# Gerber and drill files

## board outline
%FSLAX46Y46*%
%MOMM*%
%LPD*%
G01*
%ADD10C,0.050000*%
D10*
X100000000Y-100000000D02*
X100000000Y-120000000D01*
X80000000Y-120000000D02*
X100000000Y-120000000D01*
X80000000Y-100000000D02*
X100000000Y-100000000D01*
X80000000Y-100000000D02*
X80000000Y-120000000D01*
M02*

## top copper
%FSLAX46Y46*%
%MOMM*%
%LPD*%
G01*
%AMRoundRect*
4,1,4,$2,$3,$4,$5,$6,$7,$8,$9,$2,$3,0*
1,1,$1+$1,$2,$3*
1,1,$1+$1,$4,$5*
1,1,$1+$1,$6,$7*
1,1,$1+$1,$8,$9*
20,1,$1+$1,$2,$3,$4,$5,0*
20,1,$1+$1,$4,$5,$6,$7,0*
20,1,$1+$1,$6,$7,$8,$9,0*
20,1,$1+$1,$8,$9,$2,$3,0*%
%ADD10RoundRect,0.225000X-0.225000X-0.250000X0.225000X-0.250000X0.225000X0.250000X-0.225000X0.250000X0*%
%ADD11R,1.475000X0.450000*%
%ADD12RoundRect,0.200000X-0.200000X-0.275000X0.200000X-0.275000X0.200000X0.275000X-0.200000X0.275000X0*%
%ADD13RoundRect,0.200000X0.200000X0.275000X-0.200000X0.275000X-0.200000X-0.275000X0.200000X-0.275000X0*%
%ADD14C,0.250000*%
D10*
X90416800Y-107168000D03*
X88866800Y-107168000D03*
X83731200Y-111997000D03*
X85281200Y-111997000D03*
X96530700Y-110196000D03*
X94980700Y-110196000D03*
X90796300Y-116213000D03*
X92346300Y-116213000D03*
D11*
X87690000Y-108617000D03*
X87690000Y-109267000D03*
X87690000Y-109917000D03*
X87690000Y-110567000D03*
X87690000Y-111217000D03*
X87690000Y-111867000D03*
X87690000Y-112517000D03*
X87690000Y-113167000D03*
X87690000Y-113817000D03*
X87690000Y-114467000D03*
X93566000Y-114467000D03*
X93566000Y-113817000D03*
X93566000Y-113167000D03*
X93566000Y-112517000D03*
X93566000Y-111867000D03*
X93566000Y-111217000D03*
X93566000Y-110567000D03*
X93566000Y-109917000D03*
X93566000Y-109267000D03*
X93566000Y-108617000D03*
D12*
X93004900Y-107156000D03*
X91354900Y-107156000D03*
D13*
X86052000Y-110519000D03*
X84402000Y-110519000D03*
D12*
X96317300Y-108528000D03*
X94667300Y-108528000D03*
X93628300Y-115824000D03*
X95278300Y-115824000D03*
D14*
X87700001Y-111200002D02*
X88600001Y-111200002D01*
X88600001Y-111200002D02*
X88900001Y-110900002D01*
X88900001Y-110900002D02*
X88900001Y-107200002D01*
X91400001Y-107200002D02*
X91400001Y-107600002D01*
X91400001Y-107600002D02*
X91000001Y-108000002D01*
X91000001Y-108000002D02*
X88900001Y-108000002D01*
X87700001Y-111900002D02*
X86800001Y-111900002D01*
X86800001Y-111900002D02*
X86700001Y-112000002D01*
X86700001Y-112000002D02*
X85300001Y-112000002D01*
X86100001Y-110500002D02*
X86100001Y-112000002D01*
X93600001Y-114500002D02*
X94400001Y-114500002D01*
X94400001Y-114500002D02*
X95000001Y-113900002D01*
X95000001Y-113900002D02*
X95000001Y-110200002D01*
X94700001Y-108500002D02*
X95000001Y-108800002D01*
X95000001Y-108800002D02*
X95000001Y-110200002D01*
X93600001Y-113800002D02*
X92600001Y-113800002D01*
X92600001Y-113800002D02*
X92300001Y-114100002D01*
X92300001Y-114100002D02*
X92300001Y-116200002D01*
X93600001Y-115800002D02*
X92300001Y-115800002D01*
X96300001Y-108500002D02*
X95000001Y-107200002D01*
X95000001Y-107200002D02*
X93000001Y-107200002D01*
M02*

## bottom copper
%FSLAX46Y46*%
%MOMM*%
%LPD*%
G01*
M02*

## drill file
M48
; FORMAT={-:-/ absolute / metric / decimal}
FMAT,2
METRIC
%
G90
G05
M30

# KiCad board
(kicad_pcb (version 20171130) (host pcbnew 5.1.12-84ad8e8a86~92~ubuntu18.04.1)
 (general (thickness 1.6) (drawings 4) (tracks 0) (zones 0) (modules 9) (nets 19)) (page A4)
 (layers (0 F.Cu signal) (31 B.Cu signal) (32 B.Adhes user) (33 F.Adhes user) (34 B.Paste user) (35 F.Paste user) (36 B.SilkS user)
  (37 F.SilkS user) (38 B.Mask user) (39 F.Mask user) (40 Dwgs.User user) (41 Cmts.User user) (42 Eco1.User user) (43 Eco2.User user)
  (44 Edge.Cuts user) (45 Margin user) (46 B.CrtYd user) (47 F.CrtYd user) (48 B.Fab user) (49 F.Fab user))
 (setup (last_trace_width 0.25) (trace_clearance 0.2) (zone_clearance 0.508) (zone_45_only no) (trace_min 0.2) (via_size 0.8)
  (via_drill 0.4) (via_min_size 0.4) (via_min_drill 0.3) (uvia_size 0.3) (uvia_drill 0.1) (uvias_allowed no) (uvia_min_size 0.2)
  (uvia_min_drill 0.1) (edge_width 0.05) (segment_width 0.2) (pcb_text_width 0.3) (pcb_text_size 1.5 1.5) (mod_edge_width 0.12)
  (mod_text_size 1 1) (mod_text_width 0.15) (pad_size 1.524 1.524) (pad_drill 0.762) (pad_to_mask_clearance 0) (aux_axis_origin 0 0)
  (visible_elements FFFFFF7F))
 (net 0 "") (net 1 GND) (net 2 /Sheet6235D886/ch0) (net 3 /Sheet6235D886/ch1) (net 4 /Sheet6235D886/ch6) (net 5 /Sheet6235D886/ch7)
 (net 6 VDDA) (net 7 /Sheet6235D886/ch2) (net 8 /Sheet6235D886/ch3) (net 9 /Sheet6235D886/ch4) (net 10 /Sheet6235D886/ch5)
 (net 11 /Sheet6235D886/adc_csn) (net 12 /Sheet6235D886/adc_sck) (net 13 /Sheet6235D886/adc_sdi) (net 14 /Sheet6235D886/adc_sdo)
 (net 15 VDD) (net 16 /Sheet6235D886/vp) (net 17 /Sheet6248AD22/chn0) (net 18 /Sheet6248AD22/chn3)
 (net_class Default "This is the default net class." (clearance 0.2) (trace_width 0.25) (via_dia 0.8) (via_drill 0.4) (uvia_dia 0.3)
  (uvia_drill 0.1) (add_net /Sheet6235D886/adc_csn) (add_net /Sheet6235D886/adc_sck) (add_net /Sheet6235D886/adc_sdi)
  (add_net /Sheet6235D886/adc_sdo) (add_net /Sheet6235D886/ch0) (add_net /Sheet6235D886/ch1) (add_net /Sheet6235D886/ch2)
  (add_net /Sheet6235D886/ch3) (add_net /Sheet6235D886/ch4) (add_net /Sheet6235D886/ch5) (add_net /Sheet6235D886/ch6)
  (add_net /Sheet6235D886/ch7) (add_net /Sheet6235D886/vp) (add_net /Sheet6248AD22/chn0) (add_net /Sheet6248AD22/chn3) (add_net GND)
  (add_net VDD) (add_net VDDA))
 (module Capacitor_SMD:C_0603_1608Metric (layer F.Cu) (at 89.641800 107.168000)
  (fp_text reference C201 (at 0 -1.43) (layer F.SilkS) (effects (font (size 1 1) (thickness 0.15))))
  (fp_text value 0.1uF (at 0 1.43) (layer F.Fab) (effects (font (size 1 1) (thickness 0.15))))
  (pad 2 smd roundrect (at 0.775 0) (size 0.9 0.95) (layers F.Cu F.Mask F.Paste) (roundrect_rratio 0.25) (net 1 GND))
  (pad 1 smd roundrect (at -0.775 0) (size 0.9 0.95) (layers F.Cu F.Mask F.Paste) (roundrect_rratio 0.25) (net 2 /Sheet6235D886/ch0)))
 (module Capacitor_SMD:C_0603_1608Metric (layer F.Cu) (at 84.506200 111.997000)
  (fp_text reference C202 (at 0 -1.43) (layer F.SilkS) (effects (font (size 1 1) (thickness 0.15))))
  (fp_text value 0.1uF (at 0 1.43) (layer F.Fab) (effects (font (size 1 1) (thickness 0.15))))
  (pad 1 smd roundrect (at -0.775 0) (size 0.9 0.95) (layers F.Cu F.Mask F.Paste) (roundrect_rratio 0.25) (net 1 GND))
  (pad 2 smd roundrect (at 0.775 0) (size 0.9 0.95) (layers F.Cu F.Mask F.Paste) (roundrect_rratio 0.25) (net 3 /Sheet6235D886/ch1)))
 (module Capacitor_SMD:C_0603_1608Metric (layer F.Cu) (at 95.755700 110.196000)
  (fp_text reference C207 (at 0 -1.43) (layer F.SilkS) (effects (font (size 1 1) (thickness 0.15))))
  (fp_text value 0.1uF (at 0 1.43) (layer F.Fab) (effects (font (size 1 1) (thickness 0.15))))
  (pad 2 smd roundrect (at 0.775 0) (size 0.9 0.95) (layers F.Cu F.Mask F.Paste) (roundrect_rratio 0.25) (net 1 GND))
  (pad 1 smd roundrect (at -0.775 0) (size 0.9 0.95) (layers F.Cu F.Mask F.Paste) (roundrect_rratio 0.25) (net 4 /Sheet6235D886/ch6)))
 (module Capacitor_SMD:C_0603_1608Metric (layer F.Cu) (at 91.571300 116.213000)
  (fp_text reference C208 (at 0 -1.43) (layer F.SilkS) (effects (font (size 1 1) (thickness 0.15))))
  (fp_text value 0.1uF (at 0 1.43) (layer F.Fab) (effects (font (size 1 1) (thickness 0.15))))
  (pad 1 smd roundrect (at -0.775 0) (size 0.9 0.95) (layers F.Cu F.Mask F.Paste) (roundrect_rratio 0.25) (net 1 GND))
  (pad 2 smd roundrect (at 0.775 0) (size 0.9 0.95) (layers F.Cu F.Mask F.Paste) (roundrect_rratio 0.25) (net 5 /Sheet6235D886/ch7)))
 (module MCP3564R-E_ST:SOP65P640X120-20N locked (layer F.Cu) (at 90.628000 111.542000)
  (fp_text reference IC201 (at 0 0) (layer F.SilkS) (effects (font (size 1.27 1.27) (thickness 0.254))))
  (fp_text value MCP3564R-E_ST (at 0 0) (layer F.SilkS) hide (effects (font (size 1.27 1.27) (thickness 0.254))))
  (pad 1 smd rect (at -2.938 -2.925 90.000000) (size 0.45 1.475) (layers F.Cu F.Mask F.Paste) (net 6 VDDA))
  (pad 2 smd rect (at -2.938 -2.275 90.000000) (size 0.45 1.475) (layers F.Cu F.Mask F.Paste) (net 1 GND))
  (pad 3 smd rect (at -2.938 -1.625 90.000000) (size 0.45 1.475) (layers F.Cu F.Mask F.Paste) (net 1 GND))
  (pad 4 smd rect (at -2.938 -0.975 90.000000) (size 0.45 1.475) (layers F.Cu F.Mask F.Paste))
  (pad 5 smd rect (at -2.938 -0.325 90.000000) (size 0.45 1.475) (layers F.Cu F.Mask F.Paste) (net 2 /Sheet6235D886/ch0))
  (pad 6 smd rect (at -2.938 0.325 90.000000) (size 0.45 1.475) (layers F.Cu F.Mask F.Paste) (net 3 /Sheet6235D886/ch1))
  (pad 7 smd rect (at -2.938 0.975 90.000000) (size 0.45 1.475) (layers F.Cu F.Mask F.Paste) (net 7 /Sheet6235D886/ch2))
  (pad 8 smd rect (at -2.938 1.625 90.000000) (size 0.45 1.475) (layers F.Cu F.Mask F.Paste) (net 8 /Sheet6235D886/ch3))
  (pad 9 smd rect (at -2.938 2.275 90.000000) (size 0.45 1.475) (layers F.Cu F.Mask F.Paste) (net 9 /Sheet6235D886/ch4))
  (pad 10 smd rect (at -2.938 2.925 90.000000) (size 0.45 1.475) (layers F.Cu F.Mask F.Paste) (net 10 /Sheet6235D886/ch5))
  (pad 11 smd rect (at 2.938 2.925 90.000000) (size 0.45 1.475) (layers F.Cu F.Mask F.Paste) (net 4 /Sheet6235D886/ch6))
  (pad 12 smd rect (at 2.938 2.275 90.000000) (size 0.45 1.475) (layers F.Cu F.Mask F.Paste) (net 5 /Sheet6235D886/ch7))
  (pad 13 smd rect (at 2.938 1.625 90.000000) (size 0.45 1.475) (layers F.Cu F.Mask F.Paste) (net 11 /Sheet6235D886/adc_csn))
  (pad 14 smd rect (at 2.938 0.975 90.000000) (size 0.45 1.475) (layers F.Cu F.Mask F.Paste) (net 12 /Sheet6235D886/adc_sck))
  (pad 15 smd rect (at 2.938 0.325 90.000000) (size 0.45 1.475) (layers F.Cu F.Mask F.Paste) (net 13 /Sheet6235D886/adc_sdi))
  (pad 16 smd rect (at 2.938 -0.325 90.000000) (size 0.45 1.475) (layers F.Cu F.Mask F.Paste) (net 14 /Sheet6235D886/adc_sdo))
  (pad 17 smd rect (at 2.938 -0.975 90.000000) (size 0.45 1.475) (layers F.Cu F.Mask F.Paste))
  (pad 18 smd rect (at 2.938 -1.625 90.000000) (size 0.45 1.475) (layers F.Cu F.Mask F.Paste))
  (pad 19 smd rect (at 2.938 -2.275 90.000000) (size 0.45 1.475) (layers F.Cu F.Mask F.Paste) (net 1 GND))
  (pad 20 smd rect (at 2.938 -2.925 90.000000) (size 0.45 1.475) (layers F.Cu F.Mask F.Paste) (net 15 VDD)))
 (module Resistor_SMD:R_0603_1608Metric (layer F.Cu) (at 92.179900 107.156000)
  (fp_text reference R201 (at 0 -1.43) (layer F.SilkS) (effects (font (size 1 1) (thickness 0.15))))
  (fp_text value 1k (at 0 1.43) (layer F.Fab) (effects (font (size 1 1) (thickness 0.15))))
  (pad 2 smd roundrect (at 0.825 0) (size 0.8 0.95) (layers F.Cu F.Mask F.Paste) (roundrect_rratio 0.25) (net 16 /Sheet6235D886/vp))
  (pad 1 smd roundrect (at -0.825 0) (size 0.8 0.95) (layers F.Cu F.Mask F.Paste) (roundrect_rratio 0.25) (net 2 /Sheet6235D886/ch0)))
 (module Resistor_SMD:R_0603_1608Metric (layer F.Cu) (at 85.227000 110.519000 180.000000)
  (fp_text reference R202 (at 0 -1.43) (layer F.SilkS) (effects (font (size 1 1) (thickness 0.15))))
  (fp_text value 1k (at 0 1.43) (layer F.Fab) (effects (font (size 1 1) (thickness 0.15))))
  (pad 1 smd roundrect (at -0.825 0 180.000000) (size 0.8 0.95) (layers F.Cu F.Mask F.Paste) (roundrect_rratio 0.25)
   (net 3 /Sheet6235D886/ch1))
  (pad 2 smd roundrect (at 0.825 0 180.000000) (size 0.8 0.95) (layers F.Cu F.Mask F.Paste) (roundrect_rratio 0.25)
   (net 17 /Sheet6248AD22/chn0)))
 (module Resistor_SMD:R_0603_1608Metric (layer F.Cu) (at 95.492300 108.528000)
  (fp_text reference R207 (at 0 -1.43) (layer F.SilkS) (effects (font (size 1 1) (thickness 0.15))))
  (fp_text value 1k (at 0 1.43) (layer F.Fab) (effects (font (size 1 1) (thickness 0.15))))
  (pad 2 smd roundrect (at 0.825 0) (size 0.8 0.95) (layers F.Cu F.Mask F.Paste) (roundrect_rratio 0.25) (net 16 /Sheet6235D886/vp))
  (pad 1 smd roundrect (at -0.825 0) (size 0.8 0.95) (layers F.Cu F.Mask F.Paste) (roundrect_rratio 0.25) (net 4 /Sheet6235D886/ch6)))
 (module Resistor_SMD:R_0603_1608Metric (layer F.Cu) (at 94.453300 115.824000)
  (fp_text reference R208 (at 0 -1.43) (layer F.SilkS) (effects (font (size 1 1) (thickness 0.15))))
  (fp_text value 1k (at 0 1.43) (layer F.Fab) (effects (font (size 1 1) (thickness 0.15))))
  (pad 1 smd roundrect (at -0.825 0) (size 0.8 0.95) (layers F.Cu F.Mask F.Paste) (roundrect_rratio 0.25) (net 5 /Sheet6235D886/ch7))
  (pad 2 smd roundrect (at 0.825 0) (size 0.8 0.95) (layers F.Cu F.Mask F.Paste) (roundrect_rratio 0.25) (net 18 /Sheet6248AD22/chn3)))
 (gr_line (start 100 100) (end 100 120) (layer Edge.Cuts) (width 0.05))
 (gr_line (start 80 120) (end 100 120) (layer Edge.Cuts) (width 0.05))
 (gr_line (start 80 100) (end 100 100) (layer Edge.Cuts) (width 0.05))
 (gr_line (start 80 100) (end 80 120) (layer Edge.Cuts) (width 0.05))
 (segment (start 87.700001 111.200002) (end 88.600001 111.200002) (width 0.250000) (layer F.Cu) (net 2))
 (segment (start 88.600001 111.200002) (end 88.900001 110.900002) (width 0.250000) (layer F.Cu) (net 2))
 (segment (start 88.900001 110.900002) (end 88.900001 107.200002) (width 0.250000) (layer F.Cu) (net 2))
 (segment (start 91.400001 107.200002) (end 91.400001 107.600002) (width 0.250000) (layer F.Cu) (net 2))
 (segment (start 91.400001 107.600002) (end 91.000001 108.000002) (width 0.250000) (layer F.Cu) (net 2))
 (segment (start 91.000001 108.000002) (end 88.900001 108.000002) (width 0.250000) (layer F.Cu) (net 2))
 (segment (start 87.700001 111.900002) (end 86.800001 111.900002) (width 0.250000) (layer F.Cu) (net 3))
 (segment (start 86.800001 111.900002) (end 86.700001 112.000002) (width 0.250000) (layer F.Cu) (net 3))
 (segment (start 86.700001 112.000002) (end 85.300001 112.000002) (width 0.250000) (layer F.Cu) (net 3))
 (segment (start 86.100001 110.500002) (end 86.100001 112.000002) (width 0.250000) (layer F.Cu) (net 3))
 (segment (start 93.600001 114.500002) (end 94.400001 114.500002) (width 0.250000) (layer F.Cu) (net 4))
 (segment (start 94.400001 114.500002) (end 95.000001 113.900002) (width 0.250000) (layer F.Cu) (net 4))
 (segment (start 95.000001 113.900002) (end 95.000001 110.200002) (width 0.250000) (layer F.Cu) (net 4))
 (segment (start 94.700001 108.500002) (end 95.000001 108.800002) (width 0.250000) (layer F.Cu) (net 4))
 (segment (start 95.000001 108.800002) (end 95.000001 110.200002) (width 0.250000) (layer F.Cu) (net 4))
 (segment (start 93.600001 113.800002) (end 92.600001 113.800002) (width 0.250000) (layer F.Cu) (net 5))
 (segment (start 92.600001 113.800002) (end 92.300001 114.100002) (width 0.250000) (layer F.Cu) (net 5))
 (segment (start 92.300001 114.100002) (end 92.300001 116.200002) (width 0.250000) (layer F.Cu) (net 5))
 (segment (start 93.600001 115.800002) (end 92.300001 115.800002) (width 0.250000) (layer F.Cu) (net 5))
 (segment (start 96.300001 108.500002) (end 95.000001 107.200002) (width 0.250000) (layer F.Cu) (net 16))
 (segment (start 95.000001 107.200002) (end 93.000001 107.200002) (width 0.250000) (layer F.Cu) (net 16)))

